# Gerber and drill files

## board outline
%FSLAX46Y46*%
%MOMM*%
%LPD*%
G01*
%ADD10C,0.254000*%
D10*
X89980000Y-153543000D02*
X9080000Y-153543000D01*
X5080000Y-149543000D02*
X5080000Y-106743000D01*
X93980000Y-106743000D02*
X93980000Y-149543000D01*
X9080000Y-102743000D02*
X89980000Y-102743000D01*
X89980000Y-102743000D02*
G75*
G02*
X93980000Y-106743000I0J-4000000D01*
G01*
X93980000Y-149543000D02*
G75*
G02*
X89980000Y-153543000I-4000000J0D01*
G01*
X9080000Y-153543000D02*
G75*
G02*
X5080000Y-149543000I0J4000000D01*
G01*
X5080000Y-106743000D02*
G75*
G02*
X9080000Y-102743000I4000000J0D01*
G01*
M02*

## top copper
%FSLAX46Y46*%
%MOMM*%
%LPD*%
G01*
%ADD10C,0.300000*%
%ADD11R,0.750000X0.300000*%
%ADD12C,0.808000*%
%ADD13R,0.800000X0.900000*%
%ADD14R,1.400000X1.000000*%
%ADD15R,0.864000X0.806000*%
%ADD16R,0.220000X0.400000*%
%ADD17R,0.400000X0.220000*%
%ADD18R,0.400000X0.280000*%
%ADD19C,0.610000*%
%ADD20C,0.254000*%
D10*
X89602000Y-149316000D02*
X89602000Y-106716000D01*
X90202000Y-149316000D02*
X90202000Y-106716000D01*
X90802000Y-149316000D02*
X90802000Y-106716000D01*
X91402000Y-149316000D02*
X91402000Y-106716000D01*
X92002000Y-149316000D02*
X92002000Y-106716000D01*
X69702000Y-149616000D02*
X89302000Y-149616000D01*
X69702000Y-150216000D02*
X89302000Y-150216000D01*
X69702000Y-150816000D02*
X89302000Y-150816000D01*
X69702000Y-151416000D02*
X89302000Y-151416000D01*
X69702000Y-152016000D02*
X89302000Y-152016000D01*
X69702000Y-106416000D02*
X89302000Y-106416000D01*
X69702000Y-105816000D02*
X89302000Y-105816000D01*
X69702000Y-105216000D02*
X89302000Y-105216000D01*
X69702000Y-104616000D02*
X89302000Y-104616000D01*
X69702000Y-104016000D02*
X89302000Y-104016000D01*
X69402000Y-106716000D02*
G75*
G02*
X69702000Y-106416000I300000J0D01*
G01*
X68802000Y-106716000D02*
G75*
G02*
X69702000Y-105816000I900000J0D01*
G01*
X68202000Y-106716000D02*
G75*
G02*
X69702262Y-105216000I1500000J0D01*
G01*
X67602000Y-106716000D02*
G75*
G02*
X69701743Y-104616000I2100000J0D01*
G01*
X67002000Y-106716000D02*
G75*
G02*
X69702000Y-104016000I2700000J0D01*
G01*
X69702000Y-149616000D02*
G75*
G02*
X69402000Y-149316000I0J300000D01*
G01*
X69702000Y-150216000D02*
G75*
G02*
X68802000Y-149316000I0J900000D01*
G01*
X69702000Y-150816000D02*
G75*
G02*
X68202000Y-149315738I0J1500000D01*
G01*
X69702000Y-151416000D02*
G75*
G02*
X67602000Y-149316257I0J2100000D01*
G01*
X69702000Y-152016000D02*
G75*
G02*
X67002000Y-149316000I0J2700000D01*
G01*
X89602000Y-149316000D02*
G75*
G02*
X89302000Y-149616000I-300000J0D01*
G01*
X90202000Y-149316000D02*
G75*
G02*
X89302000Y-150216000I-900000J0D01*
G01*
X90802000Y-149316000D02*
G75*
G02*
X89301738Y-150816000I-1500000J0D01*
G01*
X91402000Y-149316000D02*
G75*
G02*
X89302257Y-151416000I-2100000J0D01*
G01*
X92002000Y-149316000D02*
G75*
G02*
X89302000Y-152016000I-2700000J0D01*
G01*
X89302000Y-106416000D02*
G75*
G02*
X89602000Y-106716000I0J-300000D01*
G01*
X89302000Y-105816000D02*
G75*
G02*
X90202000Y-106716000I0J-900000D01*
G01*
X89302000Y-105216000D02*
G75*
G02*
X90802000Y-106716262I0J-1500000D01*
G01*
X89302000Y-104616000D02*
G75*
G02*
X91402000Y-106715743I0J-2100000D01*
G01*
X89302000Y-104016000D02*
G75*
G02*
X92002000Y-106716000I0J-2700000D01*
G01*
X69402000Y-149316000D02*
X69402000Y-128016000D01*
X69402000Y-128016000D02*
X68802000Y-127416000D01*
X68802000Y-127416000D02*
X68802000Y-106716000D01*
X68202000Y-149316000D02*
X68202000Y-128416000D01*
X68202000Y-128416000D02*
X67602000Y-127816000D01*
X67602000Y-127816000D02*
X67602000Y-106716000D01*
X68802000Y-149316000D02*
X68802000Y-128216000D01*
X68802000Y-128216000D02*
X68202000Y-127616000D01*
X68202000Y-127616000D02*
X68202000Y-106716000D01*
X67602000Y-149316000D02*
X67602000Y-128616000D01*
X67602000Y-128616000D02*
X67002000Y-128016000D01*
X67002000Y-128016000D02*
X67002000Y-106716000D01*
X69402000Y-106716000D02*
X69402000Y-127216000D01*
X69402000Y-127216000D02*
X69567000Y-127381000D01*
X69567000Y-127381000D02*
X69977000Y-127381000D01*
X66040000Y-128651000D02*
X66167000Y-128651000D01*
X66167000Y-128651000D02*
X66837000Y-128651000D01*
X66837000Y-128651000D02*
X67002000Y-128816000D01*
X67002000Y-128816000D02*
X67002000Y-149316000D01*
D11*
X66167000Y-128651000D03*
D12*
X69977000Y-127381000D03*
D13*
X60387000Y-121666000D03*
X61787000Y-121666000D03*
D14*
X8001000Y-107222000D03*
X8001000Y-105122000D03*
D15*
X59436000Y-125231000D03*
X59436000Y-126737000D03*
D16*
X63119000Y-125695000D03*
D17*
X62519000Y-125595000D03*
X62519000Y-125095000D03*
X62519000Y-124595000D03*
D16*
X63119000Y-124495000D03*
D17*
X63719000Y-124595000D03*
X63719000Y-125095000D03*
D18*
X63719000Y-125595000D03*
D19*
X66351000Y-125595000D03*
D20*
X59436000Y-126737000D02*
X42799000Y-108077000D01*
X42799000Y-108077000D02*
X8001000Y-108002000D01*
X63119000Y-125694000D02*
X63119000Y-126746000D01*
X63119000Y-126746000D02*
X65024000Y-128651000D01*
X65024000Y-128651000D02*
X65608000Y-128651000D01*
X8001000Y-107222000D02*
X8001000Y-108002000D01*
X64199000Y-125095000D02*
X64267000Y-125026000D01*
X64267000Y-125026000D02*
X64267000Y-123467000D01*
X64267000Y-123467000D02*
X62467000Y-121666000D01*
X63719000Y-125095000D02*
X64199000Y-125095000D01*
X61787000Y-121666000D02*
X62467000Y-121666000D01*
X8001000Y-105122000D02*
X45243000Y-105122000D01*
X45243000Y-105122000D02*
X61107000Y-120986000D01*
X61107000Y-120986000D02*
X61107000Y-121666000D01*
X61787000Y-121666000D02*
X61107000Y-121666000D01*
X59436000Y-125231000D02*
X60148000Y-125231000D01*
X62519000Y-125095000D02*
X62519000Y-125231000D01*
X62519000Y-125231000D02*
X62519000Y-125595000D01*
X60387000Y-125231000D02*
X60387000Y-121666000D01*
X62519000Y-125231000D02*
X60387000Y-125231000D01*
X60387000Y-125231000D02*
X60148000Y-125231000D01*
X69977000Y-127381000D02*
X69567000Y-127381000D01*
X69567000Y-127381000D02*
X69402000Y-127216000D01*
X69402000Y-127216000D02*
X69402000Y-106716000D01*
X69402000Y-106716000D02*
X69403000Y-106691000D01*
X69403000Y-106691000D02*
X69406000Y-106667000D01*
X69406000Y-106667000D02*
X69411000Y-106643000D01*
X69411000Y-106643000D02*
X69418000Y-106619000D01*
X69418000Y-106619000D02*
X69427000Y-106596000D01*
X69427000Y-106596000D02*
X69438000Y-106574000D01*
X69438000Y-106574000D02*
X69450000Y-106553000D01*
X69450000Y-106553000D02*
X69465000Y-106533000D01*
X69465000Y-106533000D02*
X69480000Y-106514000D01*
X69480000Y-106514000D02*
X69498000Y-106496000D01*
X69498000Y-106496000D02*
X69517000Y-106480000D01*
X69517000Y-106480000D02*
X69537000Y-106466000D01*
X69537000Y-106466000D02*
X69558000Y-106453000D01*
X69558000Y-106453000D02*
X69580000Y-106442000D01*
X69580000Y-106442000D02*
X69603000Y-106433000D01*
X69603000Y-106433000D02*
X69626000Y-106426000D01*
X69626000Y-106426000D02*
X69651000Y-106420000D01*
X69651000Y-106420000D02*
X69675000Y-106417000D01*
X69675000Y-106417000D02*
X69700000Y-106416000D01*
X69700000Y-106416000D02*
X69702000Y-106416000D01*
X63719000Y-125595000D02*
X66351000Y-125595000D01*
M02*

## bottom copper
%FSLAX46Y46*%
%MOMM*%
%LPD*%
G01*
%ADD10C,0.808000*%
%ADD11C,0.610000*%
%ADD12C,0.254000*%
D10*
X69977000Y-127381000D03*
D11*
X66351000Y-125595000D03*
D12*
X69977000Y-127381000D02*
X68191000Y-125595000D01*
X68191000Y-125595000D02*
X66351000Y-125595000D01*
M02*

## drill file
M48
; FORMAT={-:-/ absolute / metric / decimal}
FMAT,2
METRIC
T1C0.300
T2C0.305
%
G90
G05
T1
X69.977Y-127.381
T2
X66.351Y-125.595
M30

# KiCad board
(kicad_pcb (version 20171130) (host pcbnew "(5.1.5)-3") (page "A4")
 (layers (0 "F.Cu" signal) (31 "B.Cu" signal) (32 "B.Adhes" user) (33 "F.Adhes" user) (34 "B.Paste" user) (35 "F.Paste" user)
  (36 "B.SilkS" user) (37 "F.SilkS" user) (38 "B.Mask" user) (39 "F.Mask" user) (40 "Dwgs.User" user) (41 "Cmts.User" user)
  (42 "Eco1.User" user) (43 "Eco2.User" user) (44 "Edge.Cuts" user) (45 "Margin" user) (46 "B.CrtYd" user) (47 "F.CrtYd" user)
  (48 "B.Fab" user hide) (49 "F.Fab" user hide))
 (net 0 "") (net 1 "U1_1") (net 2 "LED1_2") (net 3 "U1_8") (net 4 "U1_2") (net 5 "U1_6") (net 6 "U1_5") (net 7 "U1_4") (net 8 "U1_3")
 (segment (start 69.977 127.381) (end 68.191 125.595) (width 0.254) (layer "B.Cu") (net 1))
 (segment (start 68.191 125.595) (end 66.351 125.595) (width 0.254) (layer "B.Cu") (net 1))
 (gr_line (start 89.98 153.543) (end 9.08 153.543) (width 0.254) (layer "Edge.Cuts"))
 (gr_line (start 5.08 149.543) (end 5.08 106.743) (width 0.254) (layer "Edge.Cuts"))
 (gr_line (start 93.98 106.743) (end 93.98 149.543) (width 0.254) (layer "Edge.Cuts"))
 (gr_line (start 9.08 102.743) (end 89.98 102.743) (width 0.254) (layer "Edge.Cuts"))
 (gr_arc (start 89.98 106.743) (end 89.98 102.743) (angle 90) (width 0.254) (layer "Edge.Cuts"))
 (gr_arc (start 89.98 149.543) (end 93.98 149.543) (angle 90) (width 0.254) (layer "Edge.Cuts"))
 (gr_arc (start 9.08 149.543) (end 9.08 153.543) (angle 90) (width 0.254) (layer "Edge.Cuts"))
 (gr_arc (start 9.08 106.743) (end 5.08 106.743) (angle 90) (width 0.254) (layer "Edge.Cuts"))
 (segment (start 59.436 126.737) (end 42.799 108.077) (width 0.254) (layer "F.Cu") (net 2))
 (segment (start 42.799 108.077) (end 8.001 108.002) (width 0.254) (layer "F.Cu") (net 2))
 (segment (start 63.119 125.694) (end 63.119 126.746) (width 0.254) (layer "F.Cu") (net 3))
 (segment (start 63.119 126.746) (end 65.024 128.651) (width 0.254) (layer "F.Cu") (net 3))
 (segment (start 65.024 128.651) (end 65.608 128.651) (width 0.254) (layer "F.Cu") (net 3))
 (segment (start 8.001 107.222) (end 8.001 108.002) (width 0.254) (layer "F.Cu") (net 2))
 (segment (start 64.199 125.095) (end 64.267 125.026) (width 0.254) (layer "F.Cu") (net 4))
 (segment (start 64.267 125.026) (end 64.267 123.467) (width 0.254) (layer "F.Cu") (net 4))
 (segment (start 64.267 123.467) (end 62.467 121.666) (width 0.254) (layer "F.Cu") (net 4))
 (segment (start 63.719 125.095) (end 64.199 125.095) (width 0.254) (layer "F.Cu") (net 4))
 (segment (start 61.787 121.666) (end 62.467 121.666) (width 0.254) (layer "F.Cu") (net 4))
 (segment (start 8.001 105.122) (end 45.243 105.122) (width 0.254) (layer "F.Cu") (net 4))
 (segment (start 45.243 105.122) (end 61.107 120.986) (width 0.254) (layer "F.Cu") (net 4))
 (segment (start 61.107 120.986) (end 61.107 121.666) (width 0.254) (layer "F.Cu") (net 4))
 (segment (start 61.787 121.666) (end 61.107 121.666) (width 0.254) (layer "F.Cu") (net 4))
 (segment (start 59.436 125.231) (end 60.148 125.231) (width 0.254) (layer "F.Cu") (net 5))
 (segment (start 62.519 125.095) (end 62.519 125.231) (width 0.254) (layer "F.Cu") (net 5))
 (segment (start 62.519 125.231) (end 62.519 125.595) (width 0.254) (layer "F.Cu") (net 5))
 (segment (start 60.387 125.231) (end 60.387 121.666) (width 0.254) (layer "F.Cu") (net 5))
 (segment (start 62.519 125.231) (end 60.387 125.231) (width 0.254) (layer "F.Cu") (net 5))
 (segment (start 60.387 125.231) (end 60.148 125.231) (width 0.254) (layer "F.Cu") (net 5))
 (segment (start 69.977 127.381) (end 69.567 127.381) (width 0.254) (layer "F.Cu") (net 1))
 (segment (start 69.567 127.381) (end 69.402 127.216) (width 0.254) (layer "F.Cu") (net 1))
 (segment (start 69.402 127.216) (end 69.402 106.716) (width 0.254) (layer "F.Cu") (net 1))
 (segment (start 69.402 106.716) (end 69.403 106.691) (width 0.254) (layer "F.Cu") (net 1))
 (segment (start 69.403 106.691) (end 69.406 106.667) (width 0.254) (layer "F.Cu") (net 1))
 (segment (start 69.406 106.667) (end 69.411 106.643) (width 0.254) (layer "F.Cu") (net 1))
 (segment (start 69.411 106.643) (end 69.418 106.619) (width 0.254) (layer "F.Cu") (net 1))
 (segment (start 69.418 106.619) (end 69.427 106.596) (width 0.254) (layer "F.Cu") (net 1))
 (segment (start 69.427 106.596) (end 69.438 106.574) (width 0.254) (layer "F.Cu") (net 1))
 (segment (start 69.438 106.574) (end 69.45 106.553) (width 0.254) (layer "F.Cu") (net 1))
 (segment (start 69.45 106.553) (end 69.465 106.533) (width 0.254) (layer "F.Cu") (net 1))
 (segment (start 69.465 106.533) (end 69.48 106.514) (width 0.254) (layer "F.Cu") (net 1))
 (segment (start 69.48 106.514) (end 69.498 106.496) (width 0.254) (layer "F.Cu") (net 1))
 (segment (start 69.498 106.496) (end 69.517 106.48) (width 0.254) (layer "F.Cu") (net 1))
 (segment (start 69.517 106.48) (end 69.537 106.466) (width 0.254) (layer "F.Cu") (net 1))
 (segment (start 69.537 106.466) (end 69.558 106.453) (width 0.254) (layer "F.Cu") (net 1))
 (segment (start 69.558 106.453) (end 69.58 106.442) (width 0.254) (layer "F.Cu") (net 1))
 (segment (start 69.58 106.442) (end 69.603 106.433) (width 0.254) (layer "F.Cu") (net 1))
 (segment (start 69.603 106.433) (end 69.626 106.426) (width 0.254) (layer "F.Cu") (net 1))
 (segment (start 69.626 106.426) (end 69.651 106.42) (width 0.254) (layer "F.Cu") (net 1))
 (segment (start 69.651 106.42) (end 69.675 106.417) (width 0.254) (layer "F.Cu") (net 1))
 (segment (start 69.675 106.417) (end 69.7 106.416) (width 0.254) (layer "F.Cu") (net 1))
 (segment (start 69.7 106.416) (end 69.702 106.416) (width 0.254) (layer "F.Cu") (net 1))
 (segment (start 63.719 125.595) (end 66.351 125.595) (width 0.254) (layer "F.Cu") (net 1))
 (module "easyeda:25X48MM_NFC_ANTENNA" (layer "F.Cu") (at 79.502 128.016 90)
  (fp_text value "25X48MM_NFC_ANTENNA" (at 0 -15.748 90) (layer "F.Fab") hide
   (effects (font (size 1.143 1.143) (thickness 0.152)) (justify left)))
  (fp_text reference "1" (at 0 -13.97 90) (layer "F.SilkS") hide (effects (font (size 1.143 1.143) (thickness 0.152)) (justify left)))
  (fp_line (start -21.3 10.1) (end 21.3 10.1) (width 0.3) (layer "F.Cu"))
  (fp_line (start -21.3 10.7) (end 21.3 10.7) (width 0.3) (layer "F.Cu"))
  (fp_line (start -21.3 11.3) (end 21.3 11.3) (width 0.3) (layer "F.Cu"))
  (fp_line (start -21.3 11.9) (end 21.3 11.9) (width 0.3) (layer "F.Cu"))
  (fp_line (start -21.3 12.5) (end 21.3 12.5) (width 0.3) (layer "F.Cu"))
  (fp_line (start -21.6 -9.8) (end -21.6 9.8) (width 0.3) (layer "F.Cu"))
  (fp_line (start -22.2 -9.8) (end -22.2 9.8) (width 0.3) (layer "F.Cu"))
  (fp_line (start -22.8 -9.8) (end -22.8 9.8) (width 0.3) (layer "F.Cu"))
  (fp_line (start -23.4 -9.8) (end -23.4 9.8) (width 0.3) (layer "F.Cu"))
  (fp_line (start -24 -9.8) (end -24 9.8) (width 0.3) (layer "F.Cu"))
  (fp_line (start 21.6 -9.8) (end 21.6 9.8) (width 0.3) (layer "F.Cu"))
  (fp_line (start 22.2 -9.8) (end 22.2 9.8) (width 0.3) (layer "F.Cu"))
  (fp_line (start 22.8 -9.8) (end 22.8 9.8) (width 0.3) (layer "F.Cu"))
  (fp_line (start 23.4 -9.8) (end 23.4 9.8) (width 0.3) (layer "F.Cu"))
  (fp_line (start 24 -9.8) (end 24 9.8) (width 0.3) (layer "F.Cu"))
  (fp_arc (start 21.3 -9.8) (end 21.3 -10.1) (angle 90) (width 0.3) (layer "F.Cu"))
  (fp_arc (start 21.3 -9.8) (end 21.3 -10.7) (angle 90) (width 0.3) (layer "F.Cu"))
  (fp_arc (start 21.3 -9.8) (end 21.3 -11.3) (angle 90.01) (width 0.3) (layer "F.Cu"))
  (fp_arc (start 21.3 -9.8) (end 21.3 -11.9) (angle 89.993) (width 0.3) (layer "F.Cu"))
  (fp_arc (start 21.3 -9.8) (end 21.3 -12.5) (angle 90) (width 0.3) (layer "F.Cu"))
  (fp_arc (start -21.3 -9.8) (end -21.6 -9.8) (angle 90) (width 0.3) (layer "F.Cu"))
  (fp_arc (start -21.3 -9.8) (end -22.2 -9.8) (angle 90) (width 0.3) (layer "F.Cu"))
  (fp_arc (start -21.3 -9.8) (end -22.8 -9.8) (angle 90.01) (width 0.3) (layer "F.Cu"))
  (fp_arc (start -21.3 -9.8) (end -23.4 -9.8) (angle 89.993) (width 0.3) (layer "F.Cu"))
  (fp_arc (start -21.3 -9.8) (end -24 -9.8) (angle 90) (width 0.3) (layer "F.Cu"))
  (fp_arc (start -21.3 9.8) (end -21.3 10.1) (angle 90) (width 0.3) (layer "F.Cu"))
  (fp_arc (start -21.3 9.8) (end -21.3 10.7) (angle 90) (width 0.3) (layer "F.Cu"))
  (fp_arc (start -21.3 9.8) (end -21.3 11.3) (angle 90.01) (width 0.3) (layer "F.Cu"))
  (fp_arc (start -21.3 9.8) (end -21.3 11.9) (angle 89.993) (width 0.3) (layer "F.Cu"))
  (fp_arc (start -21.3 9.8) (end -21.3 12.5) (angle 90) (width 0.3) (layer "F.Cu"))
  (fp_arc (start 21.3 9.8) (end 21.6 9.8) (angle 90) (width 0.3) (layer "F.Cu"))
  (fp_arc (start 21.3 9.8) (end 22.2 9.8) (angle 90) (width 0.3) (layer "F.Cu"))
  (fp_arc (start 21.3 9.8) (end 22.8 9.8) (angle 90.01) (width 0.3) (layer "F.Cu"))
  (fp_arc (start 21.3 9.8) (end 23.4 9.8) (angle 89.993) (width 0.3) (layer "F.Cu"))
  (fp_arc (start 21.3 9.8) (end 24 9.8) (angle 90) (width 0.3) (layer "F.Cu"))
  (fp_line (start -21.3 -10.1) (end 0 -10.1) (width 0.3) (layer "F.Cu"))
  (fp_line (start 0 -10.1) (end 0.6 -10.7) (width 0.3) (layer "F.Cu"))
  (fp_line (start 0.6 -10.7) (end 21.3 -10.7) (width 0.3) (layer "F.Cu"))
  (fp_line (start -21.3 -11.3) (end -0.4 -11.3) (width 0.3) (layer "F.Cu"))
  (fp_line (start -0.4 -11.3) (end 0.2 -11.9) (width 0.3) (layer "F.Cu"))
  (fp_line (start 0.2 -11.9) (end 21.3 -11.9) (width 0.3) (layer "F.Cu"))
  (fp_line (start -21.3 -10.7) (end -0.2 -10.7) (width 0.3) (layer "F.Cu"))
  (fp_line (start -0.2 -10.7) (end 0.4 -11.3) (width 0.3) (layer "F.Cu"))
  (fp_line (start 0.4 -11.3) (end 21.3 -11.3) (width 0.3) (layer "F.Cu"))
  (fp_line (start -21.3 -11.9) (end -0.6 -11.9) (width 0.3) (layer "F.Cu"))
  (fp_line (start -0.6 -11.9) (end 0 -12.5) (width 0.3) (layer "F.Cu"))
  (fp_line (start 0 -12.5) (end 21.3 -12.5) (width 0.3) (layer "F.Cu"))
  (fp_line (start 21.3 -10.1) (end 0.8 -10.1) (width 0.3) (layer "F.Cu"))
  (fp_line (start 0.8 -10.1) (end 0.635 -9.935) (width 0.3) (layer "F.Cu"))
  (fp_line (start 0.635 -9.935) (end 0.635 -9.525) (width 0.3) (layer "F.Cu"))
  (fp_line (start -0.635 -13.462) (end -0.635 -13.335) (width 0.3) (layer "F.Cu"))
  (fp_line (start -0.635 -13.335) (end -0.635 -12.665) (width 0.3) (layer "F.Cu"))
  (fp_line (start -0.635 -12.665) (end -0.8 -12.5) (width 0.3) (layer "F.Cu"))
  (fp_line (start -0.8 -12.5) (end -21.3 -12.5) (width 0.3) (layer "F.Cu"))
  (pad "P$1" smd rect (at -0.635 -13.335 180) (size 0.75 0.3) (layers "F.Cu" "F.Paste" "F.Mask") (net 3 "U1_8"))
  (pad "P$2" thru_hole circle (at 0.635 -9.525 90) (size 0.808 0.808) (layers "*.Cu" "*.Paste" "*.Mask") (drill oval 0.3 0.3) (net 1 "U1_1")))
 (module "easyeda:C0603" (layer "F.Cu") (at 61.087 121.666 180)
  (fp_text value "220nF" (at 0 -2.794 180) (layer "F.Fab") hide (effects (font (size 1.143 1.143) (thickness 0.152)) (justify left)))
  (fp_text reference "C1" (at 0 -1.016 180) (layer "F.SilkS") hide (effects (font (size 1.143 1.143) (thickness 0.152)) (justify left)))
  (pad 2 smd rect (at 0.7 0 180) (size 0.8 0.9) (layers "F.Cu" "F.Paste" "F.Mask") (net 5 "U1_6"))
  (pad 1 smd rect (at -0.7 0 180) (size 0.8 0.9) (layers "F.Cu" "F.Paste" "F.Mask") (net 4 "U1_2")))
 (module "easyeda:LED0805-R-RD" (layer "F.Cu") (at 8.001 106.172 90)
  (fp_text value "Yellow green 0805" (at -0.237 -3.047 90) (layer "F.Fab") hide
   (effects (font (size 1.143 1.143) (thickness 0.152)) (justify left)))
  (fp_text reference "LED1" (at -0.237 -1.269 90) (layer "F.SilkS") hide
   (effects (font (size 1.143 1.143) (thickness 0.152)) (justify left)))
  (pad 2 smd rect (at -1.05 0 -90) (size 1 1.4) (layers "F.Cu" "F.Paste" "F.Mask") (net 2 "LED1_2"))
  (pad 1 smd rect (at 1.05 0 -90) (size 1 1.4) (layers "F.Cu" "F.Paste" "F.Mask") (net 4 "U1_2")))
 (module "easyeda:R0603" (layer "F.Cu") (at 59.436 125.984 90)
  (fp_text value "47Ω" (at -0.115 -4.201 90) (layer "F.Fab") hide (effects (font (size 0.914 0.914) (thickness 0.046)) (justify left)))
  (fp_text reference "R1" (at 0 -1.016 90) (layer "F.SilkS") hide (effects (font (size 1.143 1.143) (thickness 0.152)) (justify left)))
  (pad 2 smd rect (at 0.753 0 90) (size 0.806 0.864) (layers "F.Cu" "F.Paste" "F.Mask") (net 5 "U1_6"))
  (pad 1 smd rect (at -0.753 0 90) (size 0.806 0.864) (layers "F.Cu" "F.Paste" "F.Mask") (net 2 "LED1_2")))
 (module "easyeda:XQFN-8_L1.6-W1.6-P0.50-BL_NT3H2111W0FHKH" (layer "F.Cu") (at 63.119 125.095 180)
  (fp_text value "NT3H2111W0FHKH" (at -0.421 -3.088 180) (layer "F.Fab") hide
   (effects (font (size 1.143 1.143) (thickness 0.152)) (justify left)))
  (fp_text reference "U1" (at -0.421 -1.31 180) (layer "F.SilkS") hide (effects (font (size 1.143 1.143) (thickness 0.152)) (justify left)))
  (pad 8 smd rect (at 0 -0.6 -90) (size 0.4 0.22) (layers "F.Cu" "F.Paste" "F.Mask") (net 3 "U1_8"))
  (pad 7 smd rect (at 0.6 -0.5 180) (size 0.4 0.22) (layers "F.Cu" "F.Paste" "F.Mask") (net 5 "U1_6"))
  (pad 6 smd rect (at 0.6 0 180) (size 0.4 0.22) (layers "F.Cu" "F.Paste" "F.Mask") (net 5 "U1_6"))
  (pad 5 smd rect (at 0.6 0.5 180) (size 0.4 0.22) (layers "F.Cu" "F.Paste" "F.Mask") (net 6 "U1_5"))
  (pad 4 smd rect (at 0 0.6 -90) (size 0.4 0.22) (layers "F.Cu" "F.Paste" "F.Mask") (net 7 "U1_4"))
  (pad 3 smd rect (at -0.6 0.5 180) (size 0.4 0.22) (layers "F.Cu" "F.Paste" "F.Mask") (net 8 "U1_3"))
  (pad 2 smd rect (at -0.6 0 180) (size 0.4 0.22) (layers "F.Cu" "F.Paste" "F.Mask") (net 4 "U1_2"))
  (pad 1 smd rect (at -0.6 -0.5 180) (size 0.4 0.28) (layers "F.Cu" "F.Paste" "F.Mask") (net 1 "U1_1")))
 (via (at 66.351 125.595) (size 0.61) (drill 0.305) (layers "F.Cu" "B.Cu") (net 1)))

